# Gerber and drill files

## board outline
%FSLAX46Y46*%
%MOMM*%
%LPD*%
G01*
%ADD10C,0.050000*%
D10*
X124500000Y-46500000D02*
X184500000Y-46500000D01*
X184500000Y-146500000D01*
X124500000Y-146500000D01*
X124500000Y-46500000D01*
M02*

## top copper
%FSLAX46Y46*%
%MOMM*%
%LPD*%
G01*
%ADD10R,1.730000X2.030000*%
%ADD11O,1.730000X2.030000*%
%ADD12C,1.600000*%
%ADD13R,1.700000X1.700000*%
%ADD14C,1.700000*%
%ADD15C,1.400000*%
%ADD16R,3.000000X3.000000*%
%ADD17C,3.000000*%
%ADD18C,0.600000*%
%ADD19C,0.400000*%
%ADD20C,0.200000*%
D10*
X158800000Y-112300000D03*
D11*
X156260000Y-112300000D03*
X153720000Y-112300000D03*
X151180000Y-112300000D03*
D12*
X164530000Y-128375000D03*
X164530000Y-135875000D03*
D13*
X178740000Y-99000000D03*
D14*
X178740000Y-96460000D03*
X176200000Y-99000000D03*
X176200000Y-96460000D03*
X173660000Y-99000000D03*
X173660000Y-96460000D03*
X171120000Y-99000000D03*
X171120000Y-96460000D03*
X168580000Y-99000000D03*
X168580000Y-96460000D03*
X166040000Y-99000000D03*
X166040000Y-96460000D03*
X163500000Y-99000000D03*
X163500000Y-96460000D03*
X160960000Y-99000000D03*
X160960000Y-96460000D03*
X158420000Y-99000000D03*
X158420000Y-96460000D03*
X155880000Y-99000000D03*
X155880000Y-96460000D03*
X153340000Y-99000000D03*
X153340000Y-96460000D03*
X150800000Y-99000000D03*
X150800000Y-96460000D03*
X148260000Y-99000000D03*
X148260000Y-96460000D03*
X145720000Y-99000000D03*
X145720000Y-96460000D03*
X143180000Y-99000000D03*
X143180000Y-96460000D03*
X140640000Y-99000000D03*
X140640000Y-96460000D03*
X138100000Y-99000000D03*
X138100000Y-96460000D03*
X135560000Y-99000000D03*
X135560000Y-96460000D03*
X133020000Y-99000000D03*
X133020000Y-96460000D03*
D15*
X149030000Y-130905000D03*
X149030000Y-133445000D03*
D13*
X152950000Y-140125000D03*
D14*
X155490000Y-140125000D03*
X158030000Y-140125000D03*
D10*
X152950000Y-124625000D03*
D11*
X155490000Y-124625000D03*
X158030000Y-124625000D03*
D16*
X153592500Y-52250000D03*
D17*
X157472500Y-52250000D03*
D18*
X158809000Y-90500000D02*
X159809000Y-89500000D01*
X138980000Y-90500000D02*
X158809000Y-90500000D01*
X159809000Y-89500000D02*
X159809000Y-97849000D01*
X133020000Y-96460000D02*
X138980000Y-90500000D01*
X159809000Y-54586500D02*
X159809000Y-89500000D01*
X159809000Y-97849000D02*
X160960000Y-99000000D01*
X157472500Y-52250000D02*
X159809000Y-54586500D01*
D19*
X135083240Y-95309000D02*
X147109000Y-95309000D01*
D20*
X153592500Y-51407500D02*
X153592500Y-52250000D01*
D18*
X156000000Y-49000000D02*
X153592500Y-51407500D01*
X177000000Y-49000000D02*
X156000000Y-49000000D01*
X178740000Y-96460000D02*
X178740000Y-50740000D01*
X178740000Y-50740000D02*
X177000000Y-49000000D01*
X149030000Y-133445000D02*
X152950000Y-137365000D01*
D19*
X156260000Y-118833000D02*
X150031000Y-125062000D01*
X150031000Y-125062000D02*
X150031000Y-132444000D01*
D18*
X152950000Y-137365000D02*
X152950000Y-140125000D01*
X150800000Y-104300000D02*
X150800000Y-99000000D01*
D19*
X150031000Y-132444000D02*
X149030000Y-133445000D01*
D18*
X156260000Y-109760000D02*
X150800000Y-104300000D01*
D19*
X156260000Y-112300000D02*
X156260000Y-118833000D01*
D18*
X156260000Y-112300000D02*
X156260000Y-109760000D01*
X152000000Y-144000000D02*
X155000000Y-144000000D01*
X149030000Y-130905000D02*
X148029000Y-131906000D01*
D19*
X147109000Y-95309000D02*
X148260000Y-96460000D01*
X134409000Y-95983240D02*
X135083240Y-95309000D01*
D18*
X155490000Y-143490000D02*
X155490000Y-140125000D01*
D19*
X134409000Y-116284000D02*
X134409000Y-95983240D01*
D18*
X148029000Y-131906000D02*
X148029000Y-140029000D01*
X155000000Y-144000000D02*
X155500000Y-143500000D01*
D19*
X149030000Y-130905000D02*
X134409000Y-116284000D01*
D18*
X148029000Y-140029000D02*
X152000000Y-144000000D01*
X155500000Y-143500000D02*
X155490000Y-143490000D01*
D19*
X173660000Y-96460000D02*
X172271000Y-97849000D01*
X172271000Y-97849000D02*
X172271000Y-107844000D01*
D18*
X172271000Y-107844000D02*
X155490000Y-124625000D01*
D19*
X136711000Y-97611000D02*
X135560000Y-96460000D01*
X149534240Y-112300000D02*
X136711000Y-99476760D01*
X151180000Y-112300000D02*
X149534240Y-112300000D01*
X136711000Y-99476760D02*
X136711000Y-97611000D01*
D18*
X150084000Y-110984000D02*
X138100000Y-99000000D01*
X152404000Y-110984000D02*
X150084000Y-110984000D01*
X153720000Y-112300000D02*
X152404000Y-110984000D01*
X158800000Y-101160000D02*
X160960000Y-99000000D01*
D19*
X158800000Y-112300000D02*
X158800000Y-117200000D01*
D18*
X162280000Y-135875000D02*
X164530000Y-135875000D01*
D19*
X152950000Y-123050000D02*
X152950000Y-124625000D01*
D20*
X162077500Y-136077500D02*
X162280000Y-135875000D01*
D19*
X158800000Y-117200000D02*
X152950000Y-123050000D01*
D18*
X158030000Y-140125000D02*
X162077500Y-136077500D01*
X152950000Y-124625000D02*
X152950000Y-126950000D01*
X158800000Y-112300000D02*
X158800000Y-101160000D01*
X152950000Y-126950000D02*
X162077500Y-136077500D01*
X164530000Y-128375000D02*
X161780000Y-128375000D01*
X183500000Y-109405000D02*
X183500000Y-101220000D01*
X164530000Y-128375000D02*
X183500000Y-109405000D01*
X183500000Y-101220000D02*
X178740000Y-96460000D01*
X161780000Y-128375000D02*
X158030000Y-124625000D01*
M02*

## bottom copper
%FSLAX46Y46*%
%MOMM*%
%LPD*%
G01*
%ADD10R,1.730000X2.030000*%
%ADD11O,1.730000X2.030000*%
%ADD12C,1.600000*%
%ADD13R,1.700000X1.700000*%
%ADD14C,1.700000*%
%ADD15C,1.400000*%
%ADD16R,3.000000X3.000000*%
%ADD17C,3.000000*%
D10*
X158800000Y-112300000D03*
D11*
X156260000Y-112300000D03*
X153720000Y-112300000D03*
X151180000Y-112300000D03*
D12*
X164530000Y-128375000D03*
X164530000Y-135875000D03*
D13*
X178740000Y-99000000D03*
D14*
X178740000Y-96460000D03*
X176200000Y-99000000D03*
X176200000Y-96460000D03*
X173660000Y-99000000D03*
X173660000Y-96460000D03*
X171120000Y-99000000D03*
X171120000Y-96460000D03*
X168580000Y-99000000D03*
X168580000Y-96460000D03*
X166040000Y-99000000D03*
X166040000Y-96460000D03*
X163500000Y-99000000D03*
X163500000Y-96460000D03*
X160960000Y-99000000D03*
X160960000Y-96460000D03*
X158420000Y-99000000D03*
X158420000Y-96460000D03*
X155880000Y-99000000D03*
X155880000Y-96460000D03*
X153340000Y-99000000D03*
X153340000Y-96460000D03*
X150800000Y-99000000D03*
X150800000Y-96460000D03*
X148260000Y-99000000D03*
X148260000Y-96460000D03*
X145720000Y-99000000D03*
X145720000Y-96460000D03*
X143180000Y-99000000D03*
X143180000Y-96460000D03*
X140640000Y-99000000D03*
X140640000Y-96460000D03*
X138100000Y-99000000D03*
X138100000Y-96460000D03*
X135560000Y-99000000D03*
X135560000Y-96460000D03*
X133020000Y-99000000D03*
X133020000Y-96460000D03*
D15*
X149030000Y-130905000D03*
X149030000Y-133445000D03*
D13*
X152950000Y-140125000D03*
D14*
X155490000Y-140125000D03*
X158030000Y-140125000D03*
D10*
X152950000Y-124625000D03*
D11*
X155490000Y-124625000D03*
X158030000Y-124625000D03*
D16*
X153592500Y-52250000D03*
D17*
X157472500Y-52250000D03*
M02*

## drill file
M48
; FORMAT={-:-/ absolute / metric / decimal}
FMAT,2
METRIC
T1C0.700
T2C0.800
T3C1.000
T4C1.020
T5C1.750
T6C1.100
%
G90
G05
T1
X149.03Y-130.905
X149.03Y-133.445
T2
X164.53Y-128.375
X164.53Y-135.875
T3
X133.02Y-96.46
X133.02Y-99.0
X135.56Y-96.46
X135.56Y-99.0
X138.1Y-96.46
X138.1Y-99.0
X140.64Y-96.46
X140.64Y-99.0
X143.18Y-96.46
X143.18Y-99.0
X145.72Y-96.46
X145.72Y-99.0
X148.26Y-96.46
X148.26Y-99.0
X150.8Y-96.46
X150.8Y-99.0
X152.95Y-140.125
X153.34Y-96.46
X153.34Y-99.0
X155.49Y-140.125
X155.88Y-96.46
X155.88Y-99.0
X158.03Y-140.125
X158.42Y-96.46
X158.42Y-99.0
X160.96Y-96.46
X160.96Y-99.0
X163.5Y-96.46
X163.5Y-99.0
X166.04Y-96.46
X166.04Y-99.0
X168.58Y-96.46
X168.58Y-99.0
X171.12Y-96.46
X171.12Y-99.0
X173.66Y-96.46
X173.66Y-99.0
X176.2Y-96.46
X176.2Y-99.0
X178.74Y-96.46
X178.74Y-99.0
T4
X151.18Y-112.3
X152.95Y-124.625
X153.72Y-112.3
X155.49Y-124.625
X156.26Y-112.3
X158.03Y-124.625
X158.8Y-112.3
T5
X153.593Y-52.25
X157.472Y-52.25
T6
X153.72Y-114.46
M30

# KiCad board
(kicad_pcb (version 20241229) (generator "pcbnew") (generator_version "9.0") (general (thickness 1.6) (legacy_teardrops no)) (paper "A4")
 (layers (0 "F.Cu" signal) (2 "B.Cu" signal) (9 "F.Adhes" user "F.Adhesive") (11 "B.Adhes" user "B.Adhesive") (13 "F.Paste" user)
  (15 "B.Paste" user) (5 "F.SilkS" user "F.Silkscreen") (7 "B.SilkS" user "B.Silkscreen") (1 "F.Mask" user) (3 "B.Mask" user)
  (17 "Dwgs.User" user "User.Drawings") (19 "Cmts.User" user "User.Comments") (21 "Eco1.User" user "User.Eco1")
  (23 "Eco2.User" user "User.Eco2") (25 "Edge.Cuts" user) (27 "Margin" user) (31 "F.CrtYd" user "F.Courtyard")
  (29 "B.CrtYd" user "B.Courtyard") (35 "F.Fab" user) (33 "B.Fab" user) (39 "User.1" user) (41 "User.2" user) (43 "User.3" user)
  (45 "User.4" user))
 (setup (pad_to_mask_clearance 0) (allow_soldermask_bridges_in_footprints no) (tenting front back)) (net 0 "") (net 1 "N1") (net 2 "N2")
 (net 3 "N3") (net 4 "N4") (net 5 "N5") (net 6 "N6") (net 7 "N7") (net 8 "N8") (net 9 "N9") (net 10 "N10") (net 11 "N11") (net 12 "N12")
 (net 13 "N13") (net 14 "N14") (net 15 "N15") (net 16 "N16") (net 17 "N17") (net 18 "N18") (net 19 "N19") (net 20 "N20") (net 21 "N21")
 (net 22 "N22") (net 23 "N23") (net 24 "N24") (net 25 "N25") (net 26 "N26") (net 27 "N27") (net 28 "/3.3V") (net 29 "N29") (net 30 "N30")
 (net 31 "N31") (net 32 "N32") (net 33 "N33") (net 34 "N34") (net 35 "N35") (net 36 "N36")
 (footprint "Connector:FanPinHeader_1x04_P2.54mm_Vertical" (layer "F.Cu") (at 158.8 112.3 180)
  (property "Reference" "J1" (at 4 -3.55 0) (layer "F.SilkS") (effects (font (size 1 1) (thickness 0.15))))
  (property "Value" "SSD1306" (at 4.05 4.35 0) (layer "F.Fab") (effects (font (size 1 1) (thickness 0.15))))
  (pad "" np_thru_hole circle (at 5.08 -2.16 270) (size 1.1 1.1) (drill 1.1) (layers "*.Cu" "*.Mask"))
  (pad "1" thru_hole rect (at 0 0 270) (size 2.03 1.73) (drill 1.02) (layers "*.Cu" "*.Mask") (remove_unused_layers no) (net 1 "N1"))
  (pad "2" thru_hole oval (at 2.54 0 270) (size 2.03 1.73) (drill 1.02) (layers "*.Cu" "*.Mask") (remove_unused_layers no) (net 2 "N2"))
  (pad "3" thru_hole oval (at 5.08 0 270) (size 2.03 1.73) (drill 1.02) (layers "*.Cu" "*.Mask") (remove_unused_layers no) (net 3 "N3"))
  (pad "4" thru_hole oval (at 7.62 0 270) (size 2.03 1.73) (drill 1.02) (layers "*.Cu" "*.Mask") (remove_unused_layers no) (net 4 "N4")))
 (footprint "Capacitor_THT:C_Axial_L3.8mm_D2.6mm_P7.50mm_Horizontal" (layer "F.Cu") (at 164.53 128.375 -90)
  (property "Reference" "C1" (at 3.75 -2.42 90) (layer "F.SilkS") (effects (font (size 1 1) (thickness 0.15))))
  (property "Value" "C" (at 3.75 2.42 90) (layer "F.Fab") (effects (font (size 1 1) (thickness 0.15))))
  (pad "1" thru_hole circle (at 0 0 270) (size 1.6 1.6) (drill 0.8) (layers "*.Cu" "*.Mask") (remove_unused_layers no) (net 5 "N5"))
  (pad "2" thru_hole circle (at 7.5 0 270) (size 1.6 1.6) (drill 0.8) (layers "*.Cu" "*.Mask") (remove_unused_layers no) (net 1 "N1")))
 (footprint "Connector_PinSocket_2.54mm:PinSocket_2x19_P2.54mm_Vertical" (layer "F.Cu") (at 178.74 99 -90)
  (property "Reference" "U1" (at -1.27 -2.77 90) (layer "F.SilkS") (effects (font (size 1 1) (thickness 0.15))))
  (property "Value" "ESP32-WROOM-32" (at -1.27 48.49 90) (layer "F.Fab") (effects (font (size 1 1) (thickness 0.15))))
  (pad "1" thru_hole rect (at 0 0 270) (size 1.7 1.7) (drill 1) (layers "*.Cu" "*.Mask") (remove_unused_layers no) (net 1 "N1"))
  (pad "2" thru_hole circle (at -2.54 0 270) (size 1.7 1.7) (drill 1) (layers "*.Cu" "*.Mask") (remove_unused_layers no) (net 5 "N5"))
  (pad "3" thru_hole circle (at 0 2.54 270) (size 1.7 1.7) (drill 1) (layers "*.Cu" "*.Mask") (remove_unused_layers no) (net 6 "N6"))
  (pad "4" thru_hole circle (at -2.54 2.54 270) (size 1.7 1.7) (drill 1) (layers "*.Cu" "*.Mask") (remove_unused_layers no) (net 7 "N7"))
  (pad "5" thru_hole circle (at 0 5.08 270) (size 1.7 1.7) (drill 1) (layers "*.Cu" "*.Mask") (remove_unused_layers no) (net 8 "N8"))
  (pad "6" thru_hole circle (at -2.54 5.08 270) (size 1.7 1.7) (drill 1) (layers "*.Cu" "*.Mask") (remove_unused_layers no) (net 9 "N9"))
  (pad "7" thru_hole circle (at 0 7.62 270) (size 1.7 1.7) (drill 1) (layers "*.Cu" "*.Mask") (remove_unused_layers no) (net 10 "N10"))
  (pad "8" thru_hole circle (at -2.54 7.62 270) (size 1.7 1.7) (drill 1) (layers "*.Cu" "*.Mask") (remove_unused_layers no) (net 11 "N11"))
  (pad "9" thru_hole circle (at 0 10.16 270) (size 1.7 1.7) (drill 1) (layers "*.Cu" "*.Mask") (remove_unused_layers no) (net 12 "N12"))
  (pad "10" thru_hole circle (at -2.54 10.16 270) (size 1.7 1.7) (drill 1) (layers "*.Cu" "*.Mask") (remove_unused_layers no) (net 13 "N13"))
  (pad "11" thru_hole circle (at 0 12.7 270) (size 1.7 1.7) (drill 1) (layers "*.Cu" "*.Mask") (remove_unused_layers no) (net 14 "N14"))
  (pad "12" thru_hole circle (at -2.54 12.7 270) (size 1.7 1.7) (drill 1) (layers "*.Cu" "*.Mask") (remove_unused_layers no) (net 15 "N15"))
  (pad "13" thru_hole circle (at 0 15.24 270) (size 1.7 1.7) (drill 1) (layers "*.Cu" "*.Mask") (remove_unused_layers no) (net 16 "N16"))
  (pad "14" thru_hole circle (at -2.54 15.24 270) (size 1.7 1.7) (drill 1) (layers "*.Cu" "*.Mask") (remove_unused_layers no) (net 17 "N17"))
  (pad "15" thru_hole circle (at 0 17.78 270) (size 1.7 1.7) (drill 1) (layers "*.Cu" "*.Mask") (remove_unused_layers no) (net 1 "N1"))
  (pad "16" thru_hole circle (at -2.54 17.78 270) (size 1.7 1.7) (drill 1) (layers "*.Cu" "*.Mask") (remove_unused_layers no) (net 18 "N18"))
  (pad "17" thru_hole circle (at 0 20.32 270) (size 1.7 1.7) (drill 1) (layers "*.Cu" "*.Mask") (remove_unused_layers no) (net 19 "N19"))
  (pad "18" thru_hole circle (at -2.54 20.32 270) (size 1.7 1.7) (drill 1) (layers "*.Cu" "*.Mask") (remove_unused_layers no) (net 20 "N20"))
  (pad "19" thru_hole circle (at 0 22.86 270) (size 1.7 1.7) (drill 1) (layers "*.Cu" "*.Mask") (remove_unused_layers no) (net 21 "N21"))
  (pad "20" thru_hole circle (at -2.54 22.86 270) (size 1.7 1.7) (drill 1) (layers "*.Cu" "*.Mask") (remove_unused_layers no) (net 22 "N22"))
  (pad "21" thru_hole circle (at 0 25.4 270) (size 1.7 1.7) (drill 1) (layers "*.Cu" "*.Mask") (remove_unused_layers no) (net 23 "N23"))
  (pad "22" thru_hole circle (at -2.54 25.4 270) (size 1.7 1.7) (drill 1) (layers "*.Cu" "*.Mask") (remove_unused_layers no) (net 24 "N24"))
  (pad "23" thru_hole circle (at 0 27.94 270) (size 1.7 1.7) (drill 1) (layers "*.Cu" "*.Mask") (remove_unused_layers no) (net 2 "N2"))
  (pad "24" thru_hole circle (at -2.54 27.94 270) (size 1.7 1.7) (drill 1) (layers "*.Cu" "*.Mask") (remove_unused_layers no) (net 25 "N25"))
  (pad "25" thru_hole circle (at 0 30.48 270) (size 1.7 1.7) (drill 1) (layers "*.Cu" "*.Mask") (remove_unused_layers no) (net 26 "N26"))
  (pad "26" thru_hole circle (at -2.54 30.48 270) (size 1.7 1.7) (drill 1) (layers "*.Cu" "*.Mask") (remove_unused_layers no) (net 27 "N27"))
  (pad "27" thru_hole circle (at 0 33.02 270) (size 1.7 1.7) (drill 1) (layers "*.Cu" "*.Mask") (remove_unused_layers no) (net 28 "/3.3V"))
  (pad "28" thru_hole circle (at -2.54 33.02 270) (size 1.7 1.7) (drill 1) (layers "*.Cu" "*.Mask") (remove_unused_layers no) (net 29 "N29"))
  (pad "29" thru_hole circle (at 0 35.56 270) (size 1.7 1.7) (drill 1) (layers "*.Cu" "*.Mask") (remove_unused_layers no) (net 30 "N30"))
  (pad "30" thru_hole circle (at -2.54 35.56 270) (size 1.7 1.7) (drill 1) (layers "*.Cu" "*.Mask") (remove_unused_layers no) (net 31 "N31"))
  (pad "31" thru_hole circle (at 0 38.1 270) (size 1.7 1.7) (drill 1) (layers "*.Cu" "*.Mask") (remove_unused_layers no) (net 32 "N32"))
  (pad "32" thru_hole circle (at -2.54 38.1 270) (size 1.7 1.7) (drill 1) (layers "*.Cu" "*.Mask") (remove_unused_layers no) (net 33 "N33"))
  (pad "33" thru_hole circle (at 0 40.64 270) (size 1.7 1.7) (drill 1) (layers "*.Cu" "*.Mask") (remove_unused_layers no) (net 3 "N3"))
  (pad "34" thru_hole circle (at -2.54 40.64 270) (size 1.7 1.7) (drill 1) (layers "*.Cu" "*.Mask") (remove_unused_layers no) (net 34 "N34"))
  (pad "35" thru_hole circle (at 0 43.18 270) (size 1.7 1.7) (drill 1) (layers "*.Cu" "*.Mask") (remove_unused_layers no) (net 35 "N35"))
  (pad "36" thru_hole circle (at -2.54 43.18 270) (size 1.7 1.7) (drill 1) (layers "*.Cu" "*.Mask") (remove_unused_layers no) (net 4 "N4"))
  (pad "37" thru_hole circle (at 0 45.72 270) (size 1.7 1.7) (drill 1) (layers "*.Cu" "*.Mask") (remove_unused_layers no) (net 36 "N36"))
  (pad "38" thru_hole circle (at -2.54 45.72 270) (size 1.7 1.7) (drill 1) (layers "*.Cu" "*.Mask") (remove_unused_layers no) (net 1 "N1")))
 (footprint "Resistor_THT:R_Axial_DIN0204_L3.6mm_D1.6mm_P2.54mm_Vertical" (layer "F.Cu") (at 149.03 130.905 -90)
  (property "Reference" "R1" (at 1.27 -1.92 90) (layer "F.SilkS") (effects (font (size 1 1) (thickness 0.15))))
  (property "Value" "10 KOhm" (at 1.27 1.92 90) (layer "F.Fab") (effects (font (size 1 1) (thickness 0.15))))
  (pad "1" thru_hole circle (at 0 0 270) (size 1.4 1.4) (drill 0.7) (layers "*.Cu" "*.Mask") (remove_unused_layers no) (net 27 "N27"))
  (pad "2" thru_hole circle (at 2.54 0 270) (size 1.4 1.4) (drill 0.7) (layers "*.Cu" "*.Mask") (remove_unused_layers no) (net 2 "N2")))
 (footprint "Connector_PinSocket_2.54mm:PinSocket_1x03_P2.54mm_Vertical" (layer "F.Cu") (at 152.95 140.125 90)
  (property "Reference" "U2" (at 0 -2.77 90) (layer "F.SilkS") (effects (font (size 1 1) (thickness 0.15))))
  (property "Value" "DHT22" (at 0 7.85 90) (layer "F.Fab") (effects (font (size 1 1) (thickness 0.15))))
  (pad "1" thru_hole rect (at 0 0 90) (size 1.7 1.7) (drill 1) (layers "*.Cu" "*.Mask") (remove_unused_layers no) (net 2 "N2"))
  (pad "2" thru_hole circle (at 0 2.54 90) (size 1.7 1.7) (drill 1) (layers "*.Cu" "*.Mask") (remove_unused_layers no) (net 27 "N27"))
  (pad "3" thru_hole circle (at 0 5.08 90) (size 1.7 1.7) (drill 1) (layers "*.Cu" "*.Mask") (remove_unused_layers no) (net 1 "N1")))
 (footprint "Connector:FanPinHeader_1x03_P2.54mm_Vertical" (layer "F.Cu") (at 152.95 124.625)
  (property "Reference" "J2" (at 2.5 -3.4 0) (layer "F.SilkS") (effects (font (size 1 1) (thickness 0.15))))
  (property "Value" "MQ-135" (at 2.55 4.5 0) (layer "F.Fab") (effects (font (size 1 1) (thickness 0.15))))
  (pad "1" thru_hole rect (at 0 0 90) (size 2.03 1.73) (drill 1.02) (layers "*.Cu" "*.Mask") (remove_unused_layers no) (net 1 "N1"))
  (pad "2" thru_hole oval (at 2.54 0 90) (size 2.03 1.73) (drill 1.02) (layers "*.Cu" "*.Mask") (remove_unused_layers no) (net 9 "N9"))
  (pad "3" thru_hole oval (at 5.08 0 90) (size 2.03 1.73) (drill 1.02) (layers "*.Cu" "*.Mask") (remove_unused_layers no) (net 5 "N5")))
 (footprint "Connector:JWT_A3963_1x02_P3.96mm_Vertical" (layer "F.Cu") (at 153.5925 52.25)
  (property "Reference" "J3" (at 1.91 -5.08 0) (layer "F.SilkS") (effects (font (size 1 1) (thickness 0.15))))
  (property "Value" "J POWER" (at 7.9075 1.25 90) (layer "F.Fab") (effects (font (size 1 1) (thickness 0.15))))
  (pad "1" thru_hole rect (at 0 0) (size 3 3) (drill 1.75) (layers "*.Cu" "*.Mask") (remove_unused_layers no) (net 5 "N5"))
  (pad "2" thru_hole circle (at 3.88 0) (size 3 3) (drill 1.75) (layers "*.Cu" "*.Mask") (remove_unused_layers no) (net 1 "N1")))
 (gr_rect (start 124.5 46.5) (end 184.5 146.5) (stroke (width 0.05) (type solid)) (fill no) (layer "Edge.Cuts"))
 (segment (start 149.03 133.445) (end 152.95 137.365) (width 0.6) (layer "F.Cu") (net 2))
 (segment (start 156.26 118.833) (end 150.031 125.062) (width 0.4) (layer "F.Cu") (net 2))
 (segment (start 150.031 125.062) (end 150.031 132.444) (width 0.4) (layer "F.Cu") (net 2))
 (segment (start 152.95 137.365) (end 152.95 140.125) (width 0.6) (layer "F.Cu") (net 2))
 (segment (start 150.8 104.3) (end 150.8 99) (width 0.6) (layer "F.Cu") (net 2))
 (segment (start 150.031 132.444) (end 149.03 133.445) (width 0.4) (layer "F.Cu") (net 2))
 (segment (start 156.26 109.76) (end 150.8 104.3) (width 0.6) (layer "F.Cu") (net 2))
 (segment (start 156.26 112.3) (end 156.26 118.833) (width 0.4) (layer "F.Cu") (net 2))
 (segment (start 156.26 112.3) (end 156.26 109.76) (width 0.6) (layer "F.Cu") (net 2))
 (segment (start 152 144) (end 155 144) (width 0.6) (layer "F.Cu") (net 27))
 (segment (start 149.03 130.905) (end 148.029 131.906) (width 0.6) (layer "F.Cu") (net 27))
 (segment (start 147.109 95.309) (end 148.26 96.46) (width 0.4) (layer "F.Cu") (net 27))
 (segment (start 135.08324 95.309) (end 147.109 95.309) (width 0.4) (layer "F.Cu") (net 27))
 (segment (start 134.409 95.98324) (end 135.08324 95.309) (width 0.4) (layer "F.Cu") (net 27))
 (segment (start 155.49 143.49) (end 155.49 140.125) (width 0.6) (layer "F.Cu") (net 27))
 (segment (start 134.409 116.284) (end 134.409 95.98324) (width 0.4) (layer "F.Cu") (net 27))
 (segment (start 148.029 131.906) (end 148.029 140.029) (width 0.6) (layer "F.Cu") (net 27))
 (segment (start 155 144) (end 155.5 143.5) (width 0.6) (layer "F.Cu") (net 27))
 (segment (start 149.03 130.905) (end 134.409 116.284) (width 0.4) (layer "F.Cu") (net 27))
 (segment (start 148.029 140.029) (end 152 144) (width 0.6) (layer "F.Cu") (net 27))
 (segment (start 155.5 143.5) (end 155.49 143.49) (width 0.6) (layer "F.Cu") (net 27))
 (segment (start 173.66 96.46) (end 172.271 97.849) (width 0.4) (layer "F.Cu") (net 9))
 (segment (start 172.271 97.849) (end 172.271 107.844) (width 0.4) (layer "F.Cu") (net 9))
 (segment (start 172.271 107.844) (end 155.49 124.625) (width 0.6) (layer "F.Cu") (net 9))
 (segment (start 136.711 97.611) (end 135.56 96.46) (width 0.4) (layer "F.Cu") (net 4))
 (segment (start 149.53424 112.3) (end 136.711 99.47676) (width 0.4) (layer "F.Cu") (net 4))
 (segment (start 151.18 112.3) (end 149.53424 112.3) (width 0.4) (layer "F.Cu") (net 4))
 (segment (start 136.711 99.47676) (end 136.711 97.611) (width 0.4) (layer "F.Cu") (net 4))
 (segment (start 150.084 110.984) (end 138.1 99) (width 0.6) (layer "F.Cu") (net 3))
 (segment (start 152.404 110.984) (end 150.084 110.984) (width 0.6) (layer "F.Cu") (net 3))
 (segment (start 153.72 112.3) (end 152.404 110.984) (width 0.6) (layer "F.Cu") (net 3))
 (segment (start 158.8 101.16) (end 160.96 99) (width 0.6) (layer "F.Cu") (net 1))
 (segment (start 158.8 112.3) (end 158.8 117.2) (width 0.4) (layer "F.Cu") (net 1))
 (segment (start 162.28 135.875) (end 164.53 135.875) (width 0.6) (layer "F.Cu") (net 1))
 (segment (start 152.95 123.05) (end 152.95 124.625) (width 0.4) (layer "F.Cu") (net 1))
 (segment (start 159.809 97.849) (end 160.96 99) (width 0.6) (layer "F.Cu") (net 1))
 (segment (start 133.02 96.46) (end 138.98 90.5) (width 0.6) (layer "F.Cu") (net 1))
 (segment (start 162.0775 136.0775) (end 162.28 135.875) (width 0.2) (layer "F.Cu") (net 1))
 (segment (start 158.8 117.2) (end 152.95 123.05) (width 0.4) (layer "F.Cu") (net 1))
 (segment (start 158.809 90.5) (end 159.809 89.5) (width 0.6) (layer "F.Cu") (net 1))
 (segment (start 158.03 140.125) (end 162.0775 136.0775) (width 0.6) (layer "F.Cu") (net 1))
 (segment (start 152.95 124.625) (end 152.95 126.95) (width 0.6) (layer "F.Cu") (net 1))
 (segment (start 159.809 54.5865) (end 159.809 89.5) (width 0.6) (layer "F.Cu") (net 1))
 (segment (start 159.809 89.5) (end 159.809 97.849) (width 0.6) (layer "F.Cu") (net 1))
 (segment (start 138.98 90.5) (end 158.809 90.5) (width 0.6) (layer "F.Cu") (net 1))
 (segment (start 157.4725 52.25) (end 159.809 54.5865) (width 0.6) (layer "F.Cu") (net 1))
 (segment (start 158.8 112.3) (end 158.8 101.16) (width 0.6) (layer "F.Cu") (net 1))
 (segment (start 152.95 126.95) (end 162.0775 136.0775) (width 0.6) (layer "F.Cu") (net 1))
 (segment (start 156 49) (end 153.5925 51.4075) (width 0.6) (layer "F.Cu") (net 5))
 (segment (start 164.53 128.375) (end 161.78 128.375) (width 0.6) (layer "F.Cu") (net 5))
 (segment (start 178.74 50.74) (end 177 49) (width 0.6) (layer "F.Cu") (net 5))
 (segment (start 153.5925 51.4075) (end 153.5925 52.25) (width 0.2) (layer "F.Cu") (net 5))
 (segment (start 183.5 109.405) (end 183.5 101.22) (width 0.6) (layer "F.Cu") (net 5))
 (segment (start 164.53 128.375) (end 183.5 109.405) (width 0.6) (layer "F.Cu") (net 5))
 (segment (start 183.5 101.22) (end 178.74 96.46) (width 0.6) (layer "F.Cu") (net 5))
 (segment (start 178.74 96.46) (end 178.74 50.74) (width 0.6) (layer "F.Cu") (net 5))
 (segment (start 161.78 128.375) (end 158.03 124.625) (width 0.6) (layer "F.Cu") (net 5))
 (segment (start 177 49) (end 156 49) (width 0.6) (layer "F.Cu") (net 5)))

